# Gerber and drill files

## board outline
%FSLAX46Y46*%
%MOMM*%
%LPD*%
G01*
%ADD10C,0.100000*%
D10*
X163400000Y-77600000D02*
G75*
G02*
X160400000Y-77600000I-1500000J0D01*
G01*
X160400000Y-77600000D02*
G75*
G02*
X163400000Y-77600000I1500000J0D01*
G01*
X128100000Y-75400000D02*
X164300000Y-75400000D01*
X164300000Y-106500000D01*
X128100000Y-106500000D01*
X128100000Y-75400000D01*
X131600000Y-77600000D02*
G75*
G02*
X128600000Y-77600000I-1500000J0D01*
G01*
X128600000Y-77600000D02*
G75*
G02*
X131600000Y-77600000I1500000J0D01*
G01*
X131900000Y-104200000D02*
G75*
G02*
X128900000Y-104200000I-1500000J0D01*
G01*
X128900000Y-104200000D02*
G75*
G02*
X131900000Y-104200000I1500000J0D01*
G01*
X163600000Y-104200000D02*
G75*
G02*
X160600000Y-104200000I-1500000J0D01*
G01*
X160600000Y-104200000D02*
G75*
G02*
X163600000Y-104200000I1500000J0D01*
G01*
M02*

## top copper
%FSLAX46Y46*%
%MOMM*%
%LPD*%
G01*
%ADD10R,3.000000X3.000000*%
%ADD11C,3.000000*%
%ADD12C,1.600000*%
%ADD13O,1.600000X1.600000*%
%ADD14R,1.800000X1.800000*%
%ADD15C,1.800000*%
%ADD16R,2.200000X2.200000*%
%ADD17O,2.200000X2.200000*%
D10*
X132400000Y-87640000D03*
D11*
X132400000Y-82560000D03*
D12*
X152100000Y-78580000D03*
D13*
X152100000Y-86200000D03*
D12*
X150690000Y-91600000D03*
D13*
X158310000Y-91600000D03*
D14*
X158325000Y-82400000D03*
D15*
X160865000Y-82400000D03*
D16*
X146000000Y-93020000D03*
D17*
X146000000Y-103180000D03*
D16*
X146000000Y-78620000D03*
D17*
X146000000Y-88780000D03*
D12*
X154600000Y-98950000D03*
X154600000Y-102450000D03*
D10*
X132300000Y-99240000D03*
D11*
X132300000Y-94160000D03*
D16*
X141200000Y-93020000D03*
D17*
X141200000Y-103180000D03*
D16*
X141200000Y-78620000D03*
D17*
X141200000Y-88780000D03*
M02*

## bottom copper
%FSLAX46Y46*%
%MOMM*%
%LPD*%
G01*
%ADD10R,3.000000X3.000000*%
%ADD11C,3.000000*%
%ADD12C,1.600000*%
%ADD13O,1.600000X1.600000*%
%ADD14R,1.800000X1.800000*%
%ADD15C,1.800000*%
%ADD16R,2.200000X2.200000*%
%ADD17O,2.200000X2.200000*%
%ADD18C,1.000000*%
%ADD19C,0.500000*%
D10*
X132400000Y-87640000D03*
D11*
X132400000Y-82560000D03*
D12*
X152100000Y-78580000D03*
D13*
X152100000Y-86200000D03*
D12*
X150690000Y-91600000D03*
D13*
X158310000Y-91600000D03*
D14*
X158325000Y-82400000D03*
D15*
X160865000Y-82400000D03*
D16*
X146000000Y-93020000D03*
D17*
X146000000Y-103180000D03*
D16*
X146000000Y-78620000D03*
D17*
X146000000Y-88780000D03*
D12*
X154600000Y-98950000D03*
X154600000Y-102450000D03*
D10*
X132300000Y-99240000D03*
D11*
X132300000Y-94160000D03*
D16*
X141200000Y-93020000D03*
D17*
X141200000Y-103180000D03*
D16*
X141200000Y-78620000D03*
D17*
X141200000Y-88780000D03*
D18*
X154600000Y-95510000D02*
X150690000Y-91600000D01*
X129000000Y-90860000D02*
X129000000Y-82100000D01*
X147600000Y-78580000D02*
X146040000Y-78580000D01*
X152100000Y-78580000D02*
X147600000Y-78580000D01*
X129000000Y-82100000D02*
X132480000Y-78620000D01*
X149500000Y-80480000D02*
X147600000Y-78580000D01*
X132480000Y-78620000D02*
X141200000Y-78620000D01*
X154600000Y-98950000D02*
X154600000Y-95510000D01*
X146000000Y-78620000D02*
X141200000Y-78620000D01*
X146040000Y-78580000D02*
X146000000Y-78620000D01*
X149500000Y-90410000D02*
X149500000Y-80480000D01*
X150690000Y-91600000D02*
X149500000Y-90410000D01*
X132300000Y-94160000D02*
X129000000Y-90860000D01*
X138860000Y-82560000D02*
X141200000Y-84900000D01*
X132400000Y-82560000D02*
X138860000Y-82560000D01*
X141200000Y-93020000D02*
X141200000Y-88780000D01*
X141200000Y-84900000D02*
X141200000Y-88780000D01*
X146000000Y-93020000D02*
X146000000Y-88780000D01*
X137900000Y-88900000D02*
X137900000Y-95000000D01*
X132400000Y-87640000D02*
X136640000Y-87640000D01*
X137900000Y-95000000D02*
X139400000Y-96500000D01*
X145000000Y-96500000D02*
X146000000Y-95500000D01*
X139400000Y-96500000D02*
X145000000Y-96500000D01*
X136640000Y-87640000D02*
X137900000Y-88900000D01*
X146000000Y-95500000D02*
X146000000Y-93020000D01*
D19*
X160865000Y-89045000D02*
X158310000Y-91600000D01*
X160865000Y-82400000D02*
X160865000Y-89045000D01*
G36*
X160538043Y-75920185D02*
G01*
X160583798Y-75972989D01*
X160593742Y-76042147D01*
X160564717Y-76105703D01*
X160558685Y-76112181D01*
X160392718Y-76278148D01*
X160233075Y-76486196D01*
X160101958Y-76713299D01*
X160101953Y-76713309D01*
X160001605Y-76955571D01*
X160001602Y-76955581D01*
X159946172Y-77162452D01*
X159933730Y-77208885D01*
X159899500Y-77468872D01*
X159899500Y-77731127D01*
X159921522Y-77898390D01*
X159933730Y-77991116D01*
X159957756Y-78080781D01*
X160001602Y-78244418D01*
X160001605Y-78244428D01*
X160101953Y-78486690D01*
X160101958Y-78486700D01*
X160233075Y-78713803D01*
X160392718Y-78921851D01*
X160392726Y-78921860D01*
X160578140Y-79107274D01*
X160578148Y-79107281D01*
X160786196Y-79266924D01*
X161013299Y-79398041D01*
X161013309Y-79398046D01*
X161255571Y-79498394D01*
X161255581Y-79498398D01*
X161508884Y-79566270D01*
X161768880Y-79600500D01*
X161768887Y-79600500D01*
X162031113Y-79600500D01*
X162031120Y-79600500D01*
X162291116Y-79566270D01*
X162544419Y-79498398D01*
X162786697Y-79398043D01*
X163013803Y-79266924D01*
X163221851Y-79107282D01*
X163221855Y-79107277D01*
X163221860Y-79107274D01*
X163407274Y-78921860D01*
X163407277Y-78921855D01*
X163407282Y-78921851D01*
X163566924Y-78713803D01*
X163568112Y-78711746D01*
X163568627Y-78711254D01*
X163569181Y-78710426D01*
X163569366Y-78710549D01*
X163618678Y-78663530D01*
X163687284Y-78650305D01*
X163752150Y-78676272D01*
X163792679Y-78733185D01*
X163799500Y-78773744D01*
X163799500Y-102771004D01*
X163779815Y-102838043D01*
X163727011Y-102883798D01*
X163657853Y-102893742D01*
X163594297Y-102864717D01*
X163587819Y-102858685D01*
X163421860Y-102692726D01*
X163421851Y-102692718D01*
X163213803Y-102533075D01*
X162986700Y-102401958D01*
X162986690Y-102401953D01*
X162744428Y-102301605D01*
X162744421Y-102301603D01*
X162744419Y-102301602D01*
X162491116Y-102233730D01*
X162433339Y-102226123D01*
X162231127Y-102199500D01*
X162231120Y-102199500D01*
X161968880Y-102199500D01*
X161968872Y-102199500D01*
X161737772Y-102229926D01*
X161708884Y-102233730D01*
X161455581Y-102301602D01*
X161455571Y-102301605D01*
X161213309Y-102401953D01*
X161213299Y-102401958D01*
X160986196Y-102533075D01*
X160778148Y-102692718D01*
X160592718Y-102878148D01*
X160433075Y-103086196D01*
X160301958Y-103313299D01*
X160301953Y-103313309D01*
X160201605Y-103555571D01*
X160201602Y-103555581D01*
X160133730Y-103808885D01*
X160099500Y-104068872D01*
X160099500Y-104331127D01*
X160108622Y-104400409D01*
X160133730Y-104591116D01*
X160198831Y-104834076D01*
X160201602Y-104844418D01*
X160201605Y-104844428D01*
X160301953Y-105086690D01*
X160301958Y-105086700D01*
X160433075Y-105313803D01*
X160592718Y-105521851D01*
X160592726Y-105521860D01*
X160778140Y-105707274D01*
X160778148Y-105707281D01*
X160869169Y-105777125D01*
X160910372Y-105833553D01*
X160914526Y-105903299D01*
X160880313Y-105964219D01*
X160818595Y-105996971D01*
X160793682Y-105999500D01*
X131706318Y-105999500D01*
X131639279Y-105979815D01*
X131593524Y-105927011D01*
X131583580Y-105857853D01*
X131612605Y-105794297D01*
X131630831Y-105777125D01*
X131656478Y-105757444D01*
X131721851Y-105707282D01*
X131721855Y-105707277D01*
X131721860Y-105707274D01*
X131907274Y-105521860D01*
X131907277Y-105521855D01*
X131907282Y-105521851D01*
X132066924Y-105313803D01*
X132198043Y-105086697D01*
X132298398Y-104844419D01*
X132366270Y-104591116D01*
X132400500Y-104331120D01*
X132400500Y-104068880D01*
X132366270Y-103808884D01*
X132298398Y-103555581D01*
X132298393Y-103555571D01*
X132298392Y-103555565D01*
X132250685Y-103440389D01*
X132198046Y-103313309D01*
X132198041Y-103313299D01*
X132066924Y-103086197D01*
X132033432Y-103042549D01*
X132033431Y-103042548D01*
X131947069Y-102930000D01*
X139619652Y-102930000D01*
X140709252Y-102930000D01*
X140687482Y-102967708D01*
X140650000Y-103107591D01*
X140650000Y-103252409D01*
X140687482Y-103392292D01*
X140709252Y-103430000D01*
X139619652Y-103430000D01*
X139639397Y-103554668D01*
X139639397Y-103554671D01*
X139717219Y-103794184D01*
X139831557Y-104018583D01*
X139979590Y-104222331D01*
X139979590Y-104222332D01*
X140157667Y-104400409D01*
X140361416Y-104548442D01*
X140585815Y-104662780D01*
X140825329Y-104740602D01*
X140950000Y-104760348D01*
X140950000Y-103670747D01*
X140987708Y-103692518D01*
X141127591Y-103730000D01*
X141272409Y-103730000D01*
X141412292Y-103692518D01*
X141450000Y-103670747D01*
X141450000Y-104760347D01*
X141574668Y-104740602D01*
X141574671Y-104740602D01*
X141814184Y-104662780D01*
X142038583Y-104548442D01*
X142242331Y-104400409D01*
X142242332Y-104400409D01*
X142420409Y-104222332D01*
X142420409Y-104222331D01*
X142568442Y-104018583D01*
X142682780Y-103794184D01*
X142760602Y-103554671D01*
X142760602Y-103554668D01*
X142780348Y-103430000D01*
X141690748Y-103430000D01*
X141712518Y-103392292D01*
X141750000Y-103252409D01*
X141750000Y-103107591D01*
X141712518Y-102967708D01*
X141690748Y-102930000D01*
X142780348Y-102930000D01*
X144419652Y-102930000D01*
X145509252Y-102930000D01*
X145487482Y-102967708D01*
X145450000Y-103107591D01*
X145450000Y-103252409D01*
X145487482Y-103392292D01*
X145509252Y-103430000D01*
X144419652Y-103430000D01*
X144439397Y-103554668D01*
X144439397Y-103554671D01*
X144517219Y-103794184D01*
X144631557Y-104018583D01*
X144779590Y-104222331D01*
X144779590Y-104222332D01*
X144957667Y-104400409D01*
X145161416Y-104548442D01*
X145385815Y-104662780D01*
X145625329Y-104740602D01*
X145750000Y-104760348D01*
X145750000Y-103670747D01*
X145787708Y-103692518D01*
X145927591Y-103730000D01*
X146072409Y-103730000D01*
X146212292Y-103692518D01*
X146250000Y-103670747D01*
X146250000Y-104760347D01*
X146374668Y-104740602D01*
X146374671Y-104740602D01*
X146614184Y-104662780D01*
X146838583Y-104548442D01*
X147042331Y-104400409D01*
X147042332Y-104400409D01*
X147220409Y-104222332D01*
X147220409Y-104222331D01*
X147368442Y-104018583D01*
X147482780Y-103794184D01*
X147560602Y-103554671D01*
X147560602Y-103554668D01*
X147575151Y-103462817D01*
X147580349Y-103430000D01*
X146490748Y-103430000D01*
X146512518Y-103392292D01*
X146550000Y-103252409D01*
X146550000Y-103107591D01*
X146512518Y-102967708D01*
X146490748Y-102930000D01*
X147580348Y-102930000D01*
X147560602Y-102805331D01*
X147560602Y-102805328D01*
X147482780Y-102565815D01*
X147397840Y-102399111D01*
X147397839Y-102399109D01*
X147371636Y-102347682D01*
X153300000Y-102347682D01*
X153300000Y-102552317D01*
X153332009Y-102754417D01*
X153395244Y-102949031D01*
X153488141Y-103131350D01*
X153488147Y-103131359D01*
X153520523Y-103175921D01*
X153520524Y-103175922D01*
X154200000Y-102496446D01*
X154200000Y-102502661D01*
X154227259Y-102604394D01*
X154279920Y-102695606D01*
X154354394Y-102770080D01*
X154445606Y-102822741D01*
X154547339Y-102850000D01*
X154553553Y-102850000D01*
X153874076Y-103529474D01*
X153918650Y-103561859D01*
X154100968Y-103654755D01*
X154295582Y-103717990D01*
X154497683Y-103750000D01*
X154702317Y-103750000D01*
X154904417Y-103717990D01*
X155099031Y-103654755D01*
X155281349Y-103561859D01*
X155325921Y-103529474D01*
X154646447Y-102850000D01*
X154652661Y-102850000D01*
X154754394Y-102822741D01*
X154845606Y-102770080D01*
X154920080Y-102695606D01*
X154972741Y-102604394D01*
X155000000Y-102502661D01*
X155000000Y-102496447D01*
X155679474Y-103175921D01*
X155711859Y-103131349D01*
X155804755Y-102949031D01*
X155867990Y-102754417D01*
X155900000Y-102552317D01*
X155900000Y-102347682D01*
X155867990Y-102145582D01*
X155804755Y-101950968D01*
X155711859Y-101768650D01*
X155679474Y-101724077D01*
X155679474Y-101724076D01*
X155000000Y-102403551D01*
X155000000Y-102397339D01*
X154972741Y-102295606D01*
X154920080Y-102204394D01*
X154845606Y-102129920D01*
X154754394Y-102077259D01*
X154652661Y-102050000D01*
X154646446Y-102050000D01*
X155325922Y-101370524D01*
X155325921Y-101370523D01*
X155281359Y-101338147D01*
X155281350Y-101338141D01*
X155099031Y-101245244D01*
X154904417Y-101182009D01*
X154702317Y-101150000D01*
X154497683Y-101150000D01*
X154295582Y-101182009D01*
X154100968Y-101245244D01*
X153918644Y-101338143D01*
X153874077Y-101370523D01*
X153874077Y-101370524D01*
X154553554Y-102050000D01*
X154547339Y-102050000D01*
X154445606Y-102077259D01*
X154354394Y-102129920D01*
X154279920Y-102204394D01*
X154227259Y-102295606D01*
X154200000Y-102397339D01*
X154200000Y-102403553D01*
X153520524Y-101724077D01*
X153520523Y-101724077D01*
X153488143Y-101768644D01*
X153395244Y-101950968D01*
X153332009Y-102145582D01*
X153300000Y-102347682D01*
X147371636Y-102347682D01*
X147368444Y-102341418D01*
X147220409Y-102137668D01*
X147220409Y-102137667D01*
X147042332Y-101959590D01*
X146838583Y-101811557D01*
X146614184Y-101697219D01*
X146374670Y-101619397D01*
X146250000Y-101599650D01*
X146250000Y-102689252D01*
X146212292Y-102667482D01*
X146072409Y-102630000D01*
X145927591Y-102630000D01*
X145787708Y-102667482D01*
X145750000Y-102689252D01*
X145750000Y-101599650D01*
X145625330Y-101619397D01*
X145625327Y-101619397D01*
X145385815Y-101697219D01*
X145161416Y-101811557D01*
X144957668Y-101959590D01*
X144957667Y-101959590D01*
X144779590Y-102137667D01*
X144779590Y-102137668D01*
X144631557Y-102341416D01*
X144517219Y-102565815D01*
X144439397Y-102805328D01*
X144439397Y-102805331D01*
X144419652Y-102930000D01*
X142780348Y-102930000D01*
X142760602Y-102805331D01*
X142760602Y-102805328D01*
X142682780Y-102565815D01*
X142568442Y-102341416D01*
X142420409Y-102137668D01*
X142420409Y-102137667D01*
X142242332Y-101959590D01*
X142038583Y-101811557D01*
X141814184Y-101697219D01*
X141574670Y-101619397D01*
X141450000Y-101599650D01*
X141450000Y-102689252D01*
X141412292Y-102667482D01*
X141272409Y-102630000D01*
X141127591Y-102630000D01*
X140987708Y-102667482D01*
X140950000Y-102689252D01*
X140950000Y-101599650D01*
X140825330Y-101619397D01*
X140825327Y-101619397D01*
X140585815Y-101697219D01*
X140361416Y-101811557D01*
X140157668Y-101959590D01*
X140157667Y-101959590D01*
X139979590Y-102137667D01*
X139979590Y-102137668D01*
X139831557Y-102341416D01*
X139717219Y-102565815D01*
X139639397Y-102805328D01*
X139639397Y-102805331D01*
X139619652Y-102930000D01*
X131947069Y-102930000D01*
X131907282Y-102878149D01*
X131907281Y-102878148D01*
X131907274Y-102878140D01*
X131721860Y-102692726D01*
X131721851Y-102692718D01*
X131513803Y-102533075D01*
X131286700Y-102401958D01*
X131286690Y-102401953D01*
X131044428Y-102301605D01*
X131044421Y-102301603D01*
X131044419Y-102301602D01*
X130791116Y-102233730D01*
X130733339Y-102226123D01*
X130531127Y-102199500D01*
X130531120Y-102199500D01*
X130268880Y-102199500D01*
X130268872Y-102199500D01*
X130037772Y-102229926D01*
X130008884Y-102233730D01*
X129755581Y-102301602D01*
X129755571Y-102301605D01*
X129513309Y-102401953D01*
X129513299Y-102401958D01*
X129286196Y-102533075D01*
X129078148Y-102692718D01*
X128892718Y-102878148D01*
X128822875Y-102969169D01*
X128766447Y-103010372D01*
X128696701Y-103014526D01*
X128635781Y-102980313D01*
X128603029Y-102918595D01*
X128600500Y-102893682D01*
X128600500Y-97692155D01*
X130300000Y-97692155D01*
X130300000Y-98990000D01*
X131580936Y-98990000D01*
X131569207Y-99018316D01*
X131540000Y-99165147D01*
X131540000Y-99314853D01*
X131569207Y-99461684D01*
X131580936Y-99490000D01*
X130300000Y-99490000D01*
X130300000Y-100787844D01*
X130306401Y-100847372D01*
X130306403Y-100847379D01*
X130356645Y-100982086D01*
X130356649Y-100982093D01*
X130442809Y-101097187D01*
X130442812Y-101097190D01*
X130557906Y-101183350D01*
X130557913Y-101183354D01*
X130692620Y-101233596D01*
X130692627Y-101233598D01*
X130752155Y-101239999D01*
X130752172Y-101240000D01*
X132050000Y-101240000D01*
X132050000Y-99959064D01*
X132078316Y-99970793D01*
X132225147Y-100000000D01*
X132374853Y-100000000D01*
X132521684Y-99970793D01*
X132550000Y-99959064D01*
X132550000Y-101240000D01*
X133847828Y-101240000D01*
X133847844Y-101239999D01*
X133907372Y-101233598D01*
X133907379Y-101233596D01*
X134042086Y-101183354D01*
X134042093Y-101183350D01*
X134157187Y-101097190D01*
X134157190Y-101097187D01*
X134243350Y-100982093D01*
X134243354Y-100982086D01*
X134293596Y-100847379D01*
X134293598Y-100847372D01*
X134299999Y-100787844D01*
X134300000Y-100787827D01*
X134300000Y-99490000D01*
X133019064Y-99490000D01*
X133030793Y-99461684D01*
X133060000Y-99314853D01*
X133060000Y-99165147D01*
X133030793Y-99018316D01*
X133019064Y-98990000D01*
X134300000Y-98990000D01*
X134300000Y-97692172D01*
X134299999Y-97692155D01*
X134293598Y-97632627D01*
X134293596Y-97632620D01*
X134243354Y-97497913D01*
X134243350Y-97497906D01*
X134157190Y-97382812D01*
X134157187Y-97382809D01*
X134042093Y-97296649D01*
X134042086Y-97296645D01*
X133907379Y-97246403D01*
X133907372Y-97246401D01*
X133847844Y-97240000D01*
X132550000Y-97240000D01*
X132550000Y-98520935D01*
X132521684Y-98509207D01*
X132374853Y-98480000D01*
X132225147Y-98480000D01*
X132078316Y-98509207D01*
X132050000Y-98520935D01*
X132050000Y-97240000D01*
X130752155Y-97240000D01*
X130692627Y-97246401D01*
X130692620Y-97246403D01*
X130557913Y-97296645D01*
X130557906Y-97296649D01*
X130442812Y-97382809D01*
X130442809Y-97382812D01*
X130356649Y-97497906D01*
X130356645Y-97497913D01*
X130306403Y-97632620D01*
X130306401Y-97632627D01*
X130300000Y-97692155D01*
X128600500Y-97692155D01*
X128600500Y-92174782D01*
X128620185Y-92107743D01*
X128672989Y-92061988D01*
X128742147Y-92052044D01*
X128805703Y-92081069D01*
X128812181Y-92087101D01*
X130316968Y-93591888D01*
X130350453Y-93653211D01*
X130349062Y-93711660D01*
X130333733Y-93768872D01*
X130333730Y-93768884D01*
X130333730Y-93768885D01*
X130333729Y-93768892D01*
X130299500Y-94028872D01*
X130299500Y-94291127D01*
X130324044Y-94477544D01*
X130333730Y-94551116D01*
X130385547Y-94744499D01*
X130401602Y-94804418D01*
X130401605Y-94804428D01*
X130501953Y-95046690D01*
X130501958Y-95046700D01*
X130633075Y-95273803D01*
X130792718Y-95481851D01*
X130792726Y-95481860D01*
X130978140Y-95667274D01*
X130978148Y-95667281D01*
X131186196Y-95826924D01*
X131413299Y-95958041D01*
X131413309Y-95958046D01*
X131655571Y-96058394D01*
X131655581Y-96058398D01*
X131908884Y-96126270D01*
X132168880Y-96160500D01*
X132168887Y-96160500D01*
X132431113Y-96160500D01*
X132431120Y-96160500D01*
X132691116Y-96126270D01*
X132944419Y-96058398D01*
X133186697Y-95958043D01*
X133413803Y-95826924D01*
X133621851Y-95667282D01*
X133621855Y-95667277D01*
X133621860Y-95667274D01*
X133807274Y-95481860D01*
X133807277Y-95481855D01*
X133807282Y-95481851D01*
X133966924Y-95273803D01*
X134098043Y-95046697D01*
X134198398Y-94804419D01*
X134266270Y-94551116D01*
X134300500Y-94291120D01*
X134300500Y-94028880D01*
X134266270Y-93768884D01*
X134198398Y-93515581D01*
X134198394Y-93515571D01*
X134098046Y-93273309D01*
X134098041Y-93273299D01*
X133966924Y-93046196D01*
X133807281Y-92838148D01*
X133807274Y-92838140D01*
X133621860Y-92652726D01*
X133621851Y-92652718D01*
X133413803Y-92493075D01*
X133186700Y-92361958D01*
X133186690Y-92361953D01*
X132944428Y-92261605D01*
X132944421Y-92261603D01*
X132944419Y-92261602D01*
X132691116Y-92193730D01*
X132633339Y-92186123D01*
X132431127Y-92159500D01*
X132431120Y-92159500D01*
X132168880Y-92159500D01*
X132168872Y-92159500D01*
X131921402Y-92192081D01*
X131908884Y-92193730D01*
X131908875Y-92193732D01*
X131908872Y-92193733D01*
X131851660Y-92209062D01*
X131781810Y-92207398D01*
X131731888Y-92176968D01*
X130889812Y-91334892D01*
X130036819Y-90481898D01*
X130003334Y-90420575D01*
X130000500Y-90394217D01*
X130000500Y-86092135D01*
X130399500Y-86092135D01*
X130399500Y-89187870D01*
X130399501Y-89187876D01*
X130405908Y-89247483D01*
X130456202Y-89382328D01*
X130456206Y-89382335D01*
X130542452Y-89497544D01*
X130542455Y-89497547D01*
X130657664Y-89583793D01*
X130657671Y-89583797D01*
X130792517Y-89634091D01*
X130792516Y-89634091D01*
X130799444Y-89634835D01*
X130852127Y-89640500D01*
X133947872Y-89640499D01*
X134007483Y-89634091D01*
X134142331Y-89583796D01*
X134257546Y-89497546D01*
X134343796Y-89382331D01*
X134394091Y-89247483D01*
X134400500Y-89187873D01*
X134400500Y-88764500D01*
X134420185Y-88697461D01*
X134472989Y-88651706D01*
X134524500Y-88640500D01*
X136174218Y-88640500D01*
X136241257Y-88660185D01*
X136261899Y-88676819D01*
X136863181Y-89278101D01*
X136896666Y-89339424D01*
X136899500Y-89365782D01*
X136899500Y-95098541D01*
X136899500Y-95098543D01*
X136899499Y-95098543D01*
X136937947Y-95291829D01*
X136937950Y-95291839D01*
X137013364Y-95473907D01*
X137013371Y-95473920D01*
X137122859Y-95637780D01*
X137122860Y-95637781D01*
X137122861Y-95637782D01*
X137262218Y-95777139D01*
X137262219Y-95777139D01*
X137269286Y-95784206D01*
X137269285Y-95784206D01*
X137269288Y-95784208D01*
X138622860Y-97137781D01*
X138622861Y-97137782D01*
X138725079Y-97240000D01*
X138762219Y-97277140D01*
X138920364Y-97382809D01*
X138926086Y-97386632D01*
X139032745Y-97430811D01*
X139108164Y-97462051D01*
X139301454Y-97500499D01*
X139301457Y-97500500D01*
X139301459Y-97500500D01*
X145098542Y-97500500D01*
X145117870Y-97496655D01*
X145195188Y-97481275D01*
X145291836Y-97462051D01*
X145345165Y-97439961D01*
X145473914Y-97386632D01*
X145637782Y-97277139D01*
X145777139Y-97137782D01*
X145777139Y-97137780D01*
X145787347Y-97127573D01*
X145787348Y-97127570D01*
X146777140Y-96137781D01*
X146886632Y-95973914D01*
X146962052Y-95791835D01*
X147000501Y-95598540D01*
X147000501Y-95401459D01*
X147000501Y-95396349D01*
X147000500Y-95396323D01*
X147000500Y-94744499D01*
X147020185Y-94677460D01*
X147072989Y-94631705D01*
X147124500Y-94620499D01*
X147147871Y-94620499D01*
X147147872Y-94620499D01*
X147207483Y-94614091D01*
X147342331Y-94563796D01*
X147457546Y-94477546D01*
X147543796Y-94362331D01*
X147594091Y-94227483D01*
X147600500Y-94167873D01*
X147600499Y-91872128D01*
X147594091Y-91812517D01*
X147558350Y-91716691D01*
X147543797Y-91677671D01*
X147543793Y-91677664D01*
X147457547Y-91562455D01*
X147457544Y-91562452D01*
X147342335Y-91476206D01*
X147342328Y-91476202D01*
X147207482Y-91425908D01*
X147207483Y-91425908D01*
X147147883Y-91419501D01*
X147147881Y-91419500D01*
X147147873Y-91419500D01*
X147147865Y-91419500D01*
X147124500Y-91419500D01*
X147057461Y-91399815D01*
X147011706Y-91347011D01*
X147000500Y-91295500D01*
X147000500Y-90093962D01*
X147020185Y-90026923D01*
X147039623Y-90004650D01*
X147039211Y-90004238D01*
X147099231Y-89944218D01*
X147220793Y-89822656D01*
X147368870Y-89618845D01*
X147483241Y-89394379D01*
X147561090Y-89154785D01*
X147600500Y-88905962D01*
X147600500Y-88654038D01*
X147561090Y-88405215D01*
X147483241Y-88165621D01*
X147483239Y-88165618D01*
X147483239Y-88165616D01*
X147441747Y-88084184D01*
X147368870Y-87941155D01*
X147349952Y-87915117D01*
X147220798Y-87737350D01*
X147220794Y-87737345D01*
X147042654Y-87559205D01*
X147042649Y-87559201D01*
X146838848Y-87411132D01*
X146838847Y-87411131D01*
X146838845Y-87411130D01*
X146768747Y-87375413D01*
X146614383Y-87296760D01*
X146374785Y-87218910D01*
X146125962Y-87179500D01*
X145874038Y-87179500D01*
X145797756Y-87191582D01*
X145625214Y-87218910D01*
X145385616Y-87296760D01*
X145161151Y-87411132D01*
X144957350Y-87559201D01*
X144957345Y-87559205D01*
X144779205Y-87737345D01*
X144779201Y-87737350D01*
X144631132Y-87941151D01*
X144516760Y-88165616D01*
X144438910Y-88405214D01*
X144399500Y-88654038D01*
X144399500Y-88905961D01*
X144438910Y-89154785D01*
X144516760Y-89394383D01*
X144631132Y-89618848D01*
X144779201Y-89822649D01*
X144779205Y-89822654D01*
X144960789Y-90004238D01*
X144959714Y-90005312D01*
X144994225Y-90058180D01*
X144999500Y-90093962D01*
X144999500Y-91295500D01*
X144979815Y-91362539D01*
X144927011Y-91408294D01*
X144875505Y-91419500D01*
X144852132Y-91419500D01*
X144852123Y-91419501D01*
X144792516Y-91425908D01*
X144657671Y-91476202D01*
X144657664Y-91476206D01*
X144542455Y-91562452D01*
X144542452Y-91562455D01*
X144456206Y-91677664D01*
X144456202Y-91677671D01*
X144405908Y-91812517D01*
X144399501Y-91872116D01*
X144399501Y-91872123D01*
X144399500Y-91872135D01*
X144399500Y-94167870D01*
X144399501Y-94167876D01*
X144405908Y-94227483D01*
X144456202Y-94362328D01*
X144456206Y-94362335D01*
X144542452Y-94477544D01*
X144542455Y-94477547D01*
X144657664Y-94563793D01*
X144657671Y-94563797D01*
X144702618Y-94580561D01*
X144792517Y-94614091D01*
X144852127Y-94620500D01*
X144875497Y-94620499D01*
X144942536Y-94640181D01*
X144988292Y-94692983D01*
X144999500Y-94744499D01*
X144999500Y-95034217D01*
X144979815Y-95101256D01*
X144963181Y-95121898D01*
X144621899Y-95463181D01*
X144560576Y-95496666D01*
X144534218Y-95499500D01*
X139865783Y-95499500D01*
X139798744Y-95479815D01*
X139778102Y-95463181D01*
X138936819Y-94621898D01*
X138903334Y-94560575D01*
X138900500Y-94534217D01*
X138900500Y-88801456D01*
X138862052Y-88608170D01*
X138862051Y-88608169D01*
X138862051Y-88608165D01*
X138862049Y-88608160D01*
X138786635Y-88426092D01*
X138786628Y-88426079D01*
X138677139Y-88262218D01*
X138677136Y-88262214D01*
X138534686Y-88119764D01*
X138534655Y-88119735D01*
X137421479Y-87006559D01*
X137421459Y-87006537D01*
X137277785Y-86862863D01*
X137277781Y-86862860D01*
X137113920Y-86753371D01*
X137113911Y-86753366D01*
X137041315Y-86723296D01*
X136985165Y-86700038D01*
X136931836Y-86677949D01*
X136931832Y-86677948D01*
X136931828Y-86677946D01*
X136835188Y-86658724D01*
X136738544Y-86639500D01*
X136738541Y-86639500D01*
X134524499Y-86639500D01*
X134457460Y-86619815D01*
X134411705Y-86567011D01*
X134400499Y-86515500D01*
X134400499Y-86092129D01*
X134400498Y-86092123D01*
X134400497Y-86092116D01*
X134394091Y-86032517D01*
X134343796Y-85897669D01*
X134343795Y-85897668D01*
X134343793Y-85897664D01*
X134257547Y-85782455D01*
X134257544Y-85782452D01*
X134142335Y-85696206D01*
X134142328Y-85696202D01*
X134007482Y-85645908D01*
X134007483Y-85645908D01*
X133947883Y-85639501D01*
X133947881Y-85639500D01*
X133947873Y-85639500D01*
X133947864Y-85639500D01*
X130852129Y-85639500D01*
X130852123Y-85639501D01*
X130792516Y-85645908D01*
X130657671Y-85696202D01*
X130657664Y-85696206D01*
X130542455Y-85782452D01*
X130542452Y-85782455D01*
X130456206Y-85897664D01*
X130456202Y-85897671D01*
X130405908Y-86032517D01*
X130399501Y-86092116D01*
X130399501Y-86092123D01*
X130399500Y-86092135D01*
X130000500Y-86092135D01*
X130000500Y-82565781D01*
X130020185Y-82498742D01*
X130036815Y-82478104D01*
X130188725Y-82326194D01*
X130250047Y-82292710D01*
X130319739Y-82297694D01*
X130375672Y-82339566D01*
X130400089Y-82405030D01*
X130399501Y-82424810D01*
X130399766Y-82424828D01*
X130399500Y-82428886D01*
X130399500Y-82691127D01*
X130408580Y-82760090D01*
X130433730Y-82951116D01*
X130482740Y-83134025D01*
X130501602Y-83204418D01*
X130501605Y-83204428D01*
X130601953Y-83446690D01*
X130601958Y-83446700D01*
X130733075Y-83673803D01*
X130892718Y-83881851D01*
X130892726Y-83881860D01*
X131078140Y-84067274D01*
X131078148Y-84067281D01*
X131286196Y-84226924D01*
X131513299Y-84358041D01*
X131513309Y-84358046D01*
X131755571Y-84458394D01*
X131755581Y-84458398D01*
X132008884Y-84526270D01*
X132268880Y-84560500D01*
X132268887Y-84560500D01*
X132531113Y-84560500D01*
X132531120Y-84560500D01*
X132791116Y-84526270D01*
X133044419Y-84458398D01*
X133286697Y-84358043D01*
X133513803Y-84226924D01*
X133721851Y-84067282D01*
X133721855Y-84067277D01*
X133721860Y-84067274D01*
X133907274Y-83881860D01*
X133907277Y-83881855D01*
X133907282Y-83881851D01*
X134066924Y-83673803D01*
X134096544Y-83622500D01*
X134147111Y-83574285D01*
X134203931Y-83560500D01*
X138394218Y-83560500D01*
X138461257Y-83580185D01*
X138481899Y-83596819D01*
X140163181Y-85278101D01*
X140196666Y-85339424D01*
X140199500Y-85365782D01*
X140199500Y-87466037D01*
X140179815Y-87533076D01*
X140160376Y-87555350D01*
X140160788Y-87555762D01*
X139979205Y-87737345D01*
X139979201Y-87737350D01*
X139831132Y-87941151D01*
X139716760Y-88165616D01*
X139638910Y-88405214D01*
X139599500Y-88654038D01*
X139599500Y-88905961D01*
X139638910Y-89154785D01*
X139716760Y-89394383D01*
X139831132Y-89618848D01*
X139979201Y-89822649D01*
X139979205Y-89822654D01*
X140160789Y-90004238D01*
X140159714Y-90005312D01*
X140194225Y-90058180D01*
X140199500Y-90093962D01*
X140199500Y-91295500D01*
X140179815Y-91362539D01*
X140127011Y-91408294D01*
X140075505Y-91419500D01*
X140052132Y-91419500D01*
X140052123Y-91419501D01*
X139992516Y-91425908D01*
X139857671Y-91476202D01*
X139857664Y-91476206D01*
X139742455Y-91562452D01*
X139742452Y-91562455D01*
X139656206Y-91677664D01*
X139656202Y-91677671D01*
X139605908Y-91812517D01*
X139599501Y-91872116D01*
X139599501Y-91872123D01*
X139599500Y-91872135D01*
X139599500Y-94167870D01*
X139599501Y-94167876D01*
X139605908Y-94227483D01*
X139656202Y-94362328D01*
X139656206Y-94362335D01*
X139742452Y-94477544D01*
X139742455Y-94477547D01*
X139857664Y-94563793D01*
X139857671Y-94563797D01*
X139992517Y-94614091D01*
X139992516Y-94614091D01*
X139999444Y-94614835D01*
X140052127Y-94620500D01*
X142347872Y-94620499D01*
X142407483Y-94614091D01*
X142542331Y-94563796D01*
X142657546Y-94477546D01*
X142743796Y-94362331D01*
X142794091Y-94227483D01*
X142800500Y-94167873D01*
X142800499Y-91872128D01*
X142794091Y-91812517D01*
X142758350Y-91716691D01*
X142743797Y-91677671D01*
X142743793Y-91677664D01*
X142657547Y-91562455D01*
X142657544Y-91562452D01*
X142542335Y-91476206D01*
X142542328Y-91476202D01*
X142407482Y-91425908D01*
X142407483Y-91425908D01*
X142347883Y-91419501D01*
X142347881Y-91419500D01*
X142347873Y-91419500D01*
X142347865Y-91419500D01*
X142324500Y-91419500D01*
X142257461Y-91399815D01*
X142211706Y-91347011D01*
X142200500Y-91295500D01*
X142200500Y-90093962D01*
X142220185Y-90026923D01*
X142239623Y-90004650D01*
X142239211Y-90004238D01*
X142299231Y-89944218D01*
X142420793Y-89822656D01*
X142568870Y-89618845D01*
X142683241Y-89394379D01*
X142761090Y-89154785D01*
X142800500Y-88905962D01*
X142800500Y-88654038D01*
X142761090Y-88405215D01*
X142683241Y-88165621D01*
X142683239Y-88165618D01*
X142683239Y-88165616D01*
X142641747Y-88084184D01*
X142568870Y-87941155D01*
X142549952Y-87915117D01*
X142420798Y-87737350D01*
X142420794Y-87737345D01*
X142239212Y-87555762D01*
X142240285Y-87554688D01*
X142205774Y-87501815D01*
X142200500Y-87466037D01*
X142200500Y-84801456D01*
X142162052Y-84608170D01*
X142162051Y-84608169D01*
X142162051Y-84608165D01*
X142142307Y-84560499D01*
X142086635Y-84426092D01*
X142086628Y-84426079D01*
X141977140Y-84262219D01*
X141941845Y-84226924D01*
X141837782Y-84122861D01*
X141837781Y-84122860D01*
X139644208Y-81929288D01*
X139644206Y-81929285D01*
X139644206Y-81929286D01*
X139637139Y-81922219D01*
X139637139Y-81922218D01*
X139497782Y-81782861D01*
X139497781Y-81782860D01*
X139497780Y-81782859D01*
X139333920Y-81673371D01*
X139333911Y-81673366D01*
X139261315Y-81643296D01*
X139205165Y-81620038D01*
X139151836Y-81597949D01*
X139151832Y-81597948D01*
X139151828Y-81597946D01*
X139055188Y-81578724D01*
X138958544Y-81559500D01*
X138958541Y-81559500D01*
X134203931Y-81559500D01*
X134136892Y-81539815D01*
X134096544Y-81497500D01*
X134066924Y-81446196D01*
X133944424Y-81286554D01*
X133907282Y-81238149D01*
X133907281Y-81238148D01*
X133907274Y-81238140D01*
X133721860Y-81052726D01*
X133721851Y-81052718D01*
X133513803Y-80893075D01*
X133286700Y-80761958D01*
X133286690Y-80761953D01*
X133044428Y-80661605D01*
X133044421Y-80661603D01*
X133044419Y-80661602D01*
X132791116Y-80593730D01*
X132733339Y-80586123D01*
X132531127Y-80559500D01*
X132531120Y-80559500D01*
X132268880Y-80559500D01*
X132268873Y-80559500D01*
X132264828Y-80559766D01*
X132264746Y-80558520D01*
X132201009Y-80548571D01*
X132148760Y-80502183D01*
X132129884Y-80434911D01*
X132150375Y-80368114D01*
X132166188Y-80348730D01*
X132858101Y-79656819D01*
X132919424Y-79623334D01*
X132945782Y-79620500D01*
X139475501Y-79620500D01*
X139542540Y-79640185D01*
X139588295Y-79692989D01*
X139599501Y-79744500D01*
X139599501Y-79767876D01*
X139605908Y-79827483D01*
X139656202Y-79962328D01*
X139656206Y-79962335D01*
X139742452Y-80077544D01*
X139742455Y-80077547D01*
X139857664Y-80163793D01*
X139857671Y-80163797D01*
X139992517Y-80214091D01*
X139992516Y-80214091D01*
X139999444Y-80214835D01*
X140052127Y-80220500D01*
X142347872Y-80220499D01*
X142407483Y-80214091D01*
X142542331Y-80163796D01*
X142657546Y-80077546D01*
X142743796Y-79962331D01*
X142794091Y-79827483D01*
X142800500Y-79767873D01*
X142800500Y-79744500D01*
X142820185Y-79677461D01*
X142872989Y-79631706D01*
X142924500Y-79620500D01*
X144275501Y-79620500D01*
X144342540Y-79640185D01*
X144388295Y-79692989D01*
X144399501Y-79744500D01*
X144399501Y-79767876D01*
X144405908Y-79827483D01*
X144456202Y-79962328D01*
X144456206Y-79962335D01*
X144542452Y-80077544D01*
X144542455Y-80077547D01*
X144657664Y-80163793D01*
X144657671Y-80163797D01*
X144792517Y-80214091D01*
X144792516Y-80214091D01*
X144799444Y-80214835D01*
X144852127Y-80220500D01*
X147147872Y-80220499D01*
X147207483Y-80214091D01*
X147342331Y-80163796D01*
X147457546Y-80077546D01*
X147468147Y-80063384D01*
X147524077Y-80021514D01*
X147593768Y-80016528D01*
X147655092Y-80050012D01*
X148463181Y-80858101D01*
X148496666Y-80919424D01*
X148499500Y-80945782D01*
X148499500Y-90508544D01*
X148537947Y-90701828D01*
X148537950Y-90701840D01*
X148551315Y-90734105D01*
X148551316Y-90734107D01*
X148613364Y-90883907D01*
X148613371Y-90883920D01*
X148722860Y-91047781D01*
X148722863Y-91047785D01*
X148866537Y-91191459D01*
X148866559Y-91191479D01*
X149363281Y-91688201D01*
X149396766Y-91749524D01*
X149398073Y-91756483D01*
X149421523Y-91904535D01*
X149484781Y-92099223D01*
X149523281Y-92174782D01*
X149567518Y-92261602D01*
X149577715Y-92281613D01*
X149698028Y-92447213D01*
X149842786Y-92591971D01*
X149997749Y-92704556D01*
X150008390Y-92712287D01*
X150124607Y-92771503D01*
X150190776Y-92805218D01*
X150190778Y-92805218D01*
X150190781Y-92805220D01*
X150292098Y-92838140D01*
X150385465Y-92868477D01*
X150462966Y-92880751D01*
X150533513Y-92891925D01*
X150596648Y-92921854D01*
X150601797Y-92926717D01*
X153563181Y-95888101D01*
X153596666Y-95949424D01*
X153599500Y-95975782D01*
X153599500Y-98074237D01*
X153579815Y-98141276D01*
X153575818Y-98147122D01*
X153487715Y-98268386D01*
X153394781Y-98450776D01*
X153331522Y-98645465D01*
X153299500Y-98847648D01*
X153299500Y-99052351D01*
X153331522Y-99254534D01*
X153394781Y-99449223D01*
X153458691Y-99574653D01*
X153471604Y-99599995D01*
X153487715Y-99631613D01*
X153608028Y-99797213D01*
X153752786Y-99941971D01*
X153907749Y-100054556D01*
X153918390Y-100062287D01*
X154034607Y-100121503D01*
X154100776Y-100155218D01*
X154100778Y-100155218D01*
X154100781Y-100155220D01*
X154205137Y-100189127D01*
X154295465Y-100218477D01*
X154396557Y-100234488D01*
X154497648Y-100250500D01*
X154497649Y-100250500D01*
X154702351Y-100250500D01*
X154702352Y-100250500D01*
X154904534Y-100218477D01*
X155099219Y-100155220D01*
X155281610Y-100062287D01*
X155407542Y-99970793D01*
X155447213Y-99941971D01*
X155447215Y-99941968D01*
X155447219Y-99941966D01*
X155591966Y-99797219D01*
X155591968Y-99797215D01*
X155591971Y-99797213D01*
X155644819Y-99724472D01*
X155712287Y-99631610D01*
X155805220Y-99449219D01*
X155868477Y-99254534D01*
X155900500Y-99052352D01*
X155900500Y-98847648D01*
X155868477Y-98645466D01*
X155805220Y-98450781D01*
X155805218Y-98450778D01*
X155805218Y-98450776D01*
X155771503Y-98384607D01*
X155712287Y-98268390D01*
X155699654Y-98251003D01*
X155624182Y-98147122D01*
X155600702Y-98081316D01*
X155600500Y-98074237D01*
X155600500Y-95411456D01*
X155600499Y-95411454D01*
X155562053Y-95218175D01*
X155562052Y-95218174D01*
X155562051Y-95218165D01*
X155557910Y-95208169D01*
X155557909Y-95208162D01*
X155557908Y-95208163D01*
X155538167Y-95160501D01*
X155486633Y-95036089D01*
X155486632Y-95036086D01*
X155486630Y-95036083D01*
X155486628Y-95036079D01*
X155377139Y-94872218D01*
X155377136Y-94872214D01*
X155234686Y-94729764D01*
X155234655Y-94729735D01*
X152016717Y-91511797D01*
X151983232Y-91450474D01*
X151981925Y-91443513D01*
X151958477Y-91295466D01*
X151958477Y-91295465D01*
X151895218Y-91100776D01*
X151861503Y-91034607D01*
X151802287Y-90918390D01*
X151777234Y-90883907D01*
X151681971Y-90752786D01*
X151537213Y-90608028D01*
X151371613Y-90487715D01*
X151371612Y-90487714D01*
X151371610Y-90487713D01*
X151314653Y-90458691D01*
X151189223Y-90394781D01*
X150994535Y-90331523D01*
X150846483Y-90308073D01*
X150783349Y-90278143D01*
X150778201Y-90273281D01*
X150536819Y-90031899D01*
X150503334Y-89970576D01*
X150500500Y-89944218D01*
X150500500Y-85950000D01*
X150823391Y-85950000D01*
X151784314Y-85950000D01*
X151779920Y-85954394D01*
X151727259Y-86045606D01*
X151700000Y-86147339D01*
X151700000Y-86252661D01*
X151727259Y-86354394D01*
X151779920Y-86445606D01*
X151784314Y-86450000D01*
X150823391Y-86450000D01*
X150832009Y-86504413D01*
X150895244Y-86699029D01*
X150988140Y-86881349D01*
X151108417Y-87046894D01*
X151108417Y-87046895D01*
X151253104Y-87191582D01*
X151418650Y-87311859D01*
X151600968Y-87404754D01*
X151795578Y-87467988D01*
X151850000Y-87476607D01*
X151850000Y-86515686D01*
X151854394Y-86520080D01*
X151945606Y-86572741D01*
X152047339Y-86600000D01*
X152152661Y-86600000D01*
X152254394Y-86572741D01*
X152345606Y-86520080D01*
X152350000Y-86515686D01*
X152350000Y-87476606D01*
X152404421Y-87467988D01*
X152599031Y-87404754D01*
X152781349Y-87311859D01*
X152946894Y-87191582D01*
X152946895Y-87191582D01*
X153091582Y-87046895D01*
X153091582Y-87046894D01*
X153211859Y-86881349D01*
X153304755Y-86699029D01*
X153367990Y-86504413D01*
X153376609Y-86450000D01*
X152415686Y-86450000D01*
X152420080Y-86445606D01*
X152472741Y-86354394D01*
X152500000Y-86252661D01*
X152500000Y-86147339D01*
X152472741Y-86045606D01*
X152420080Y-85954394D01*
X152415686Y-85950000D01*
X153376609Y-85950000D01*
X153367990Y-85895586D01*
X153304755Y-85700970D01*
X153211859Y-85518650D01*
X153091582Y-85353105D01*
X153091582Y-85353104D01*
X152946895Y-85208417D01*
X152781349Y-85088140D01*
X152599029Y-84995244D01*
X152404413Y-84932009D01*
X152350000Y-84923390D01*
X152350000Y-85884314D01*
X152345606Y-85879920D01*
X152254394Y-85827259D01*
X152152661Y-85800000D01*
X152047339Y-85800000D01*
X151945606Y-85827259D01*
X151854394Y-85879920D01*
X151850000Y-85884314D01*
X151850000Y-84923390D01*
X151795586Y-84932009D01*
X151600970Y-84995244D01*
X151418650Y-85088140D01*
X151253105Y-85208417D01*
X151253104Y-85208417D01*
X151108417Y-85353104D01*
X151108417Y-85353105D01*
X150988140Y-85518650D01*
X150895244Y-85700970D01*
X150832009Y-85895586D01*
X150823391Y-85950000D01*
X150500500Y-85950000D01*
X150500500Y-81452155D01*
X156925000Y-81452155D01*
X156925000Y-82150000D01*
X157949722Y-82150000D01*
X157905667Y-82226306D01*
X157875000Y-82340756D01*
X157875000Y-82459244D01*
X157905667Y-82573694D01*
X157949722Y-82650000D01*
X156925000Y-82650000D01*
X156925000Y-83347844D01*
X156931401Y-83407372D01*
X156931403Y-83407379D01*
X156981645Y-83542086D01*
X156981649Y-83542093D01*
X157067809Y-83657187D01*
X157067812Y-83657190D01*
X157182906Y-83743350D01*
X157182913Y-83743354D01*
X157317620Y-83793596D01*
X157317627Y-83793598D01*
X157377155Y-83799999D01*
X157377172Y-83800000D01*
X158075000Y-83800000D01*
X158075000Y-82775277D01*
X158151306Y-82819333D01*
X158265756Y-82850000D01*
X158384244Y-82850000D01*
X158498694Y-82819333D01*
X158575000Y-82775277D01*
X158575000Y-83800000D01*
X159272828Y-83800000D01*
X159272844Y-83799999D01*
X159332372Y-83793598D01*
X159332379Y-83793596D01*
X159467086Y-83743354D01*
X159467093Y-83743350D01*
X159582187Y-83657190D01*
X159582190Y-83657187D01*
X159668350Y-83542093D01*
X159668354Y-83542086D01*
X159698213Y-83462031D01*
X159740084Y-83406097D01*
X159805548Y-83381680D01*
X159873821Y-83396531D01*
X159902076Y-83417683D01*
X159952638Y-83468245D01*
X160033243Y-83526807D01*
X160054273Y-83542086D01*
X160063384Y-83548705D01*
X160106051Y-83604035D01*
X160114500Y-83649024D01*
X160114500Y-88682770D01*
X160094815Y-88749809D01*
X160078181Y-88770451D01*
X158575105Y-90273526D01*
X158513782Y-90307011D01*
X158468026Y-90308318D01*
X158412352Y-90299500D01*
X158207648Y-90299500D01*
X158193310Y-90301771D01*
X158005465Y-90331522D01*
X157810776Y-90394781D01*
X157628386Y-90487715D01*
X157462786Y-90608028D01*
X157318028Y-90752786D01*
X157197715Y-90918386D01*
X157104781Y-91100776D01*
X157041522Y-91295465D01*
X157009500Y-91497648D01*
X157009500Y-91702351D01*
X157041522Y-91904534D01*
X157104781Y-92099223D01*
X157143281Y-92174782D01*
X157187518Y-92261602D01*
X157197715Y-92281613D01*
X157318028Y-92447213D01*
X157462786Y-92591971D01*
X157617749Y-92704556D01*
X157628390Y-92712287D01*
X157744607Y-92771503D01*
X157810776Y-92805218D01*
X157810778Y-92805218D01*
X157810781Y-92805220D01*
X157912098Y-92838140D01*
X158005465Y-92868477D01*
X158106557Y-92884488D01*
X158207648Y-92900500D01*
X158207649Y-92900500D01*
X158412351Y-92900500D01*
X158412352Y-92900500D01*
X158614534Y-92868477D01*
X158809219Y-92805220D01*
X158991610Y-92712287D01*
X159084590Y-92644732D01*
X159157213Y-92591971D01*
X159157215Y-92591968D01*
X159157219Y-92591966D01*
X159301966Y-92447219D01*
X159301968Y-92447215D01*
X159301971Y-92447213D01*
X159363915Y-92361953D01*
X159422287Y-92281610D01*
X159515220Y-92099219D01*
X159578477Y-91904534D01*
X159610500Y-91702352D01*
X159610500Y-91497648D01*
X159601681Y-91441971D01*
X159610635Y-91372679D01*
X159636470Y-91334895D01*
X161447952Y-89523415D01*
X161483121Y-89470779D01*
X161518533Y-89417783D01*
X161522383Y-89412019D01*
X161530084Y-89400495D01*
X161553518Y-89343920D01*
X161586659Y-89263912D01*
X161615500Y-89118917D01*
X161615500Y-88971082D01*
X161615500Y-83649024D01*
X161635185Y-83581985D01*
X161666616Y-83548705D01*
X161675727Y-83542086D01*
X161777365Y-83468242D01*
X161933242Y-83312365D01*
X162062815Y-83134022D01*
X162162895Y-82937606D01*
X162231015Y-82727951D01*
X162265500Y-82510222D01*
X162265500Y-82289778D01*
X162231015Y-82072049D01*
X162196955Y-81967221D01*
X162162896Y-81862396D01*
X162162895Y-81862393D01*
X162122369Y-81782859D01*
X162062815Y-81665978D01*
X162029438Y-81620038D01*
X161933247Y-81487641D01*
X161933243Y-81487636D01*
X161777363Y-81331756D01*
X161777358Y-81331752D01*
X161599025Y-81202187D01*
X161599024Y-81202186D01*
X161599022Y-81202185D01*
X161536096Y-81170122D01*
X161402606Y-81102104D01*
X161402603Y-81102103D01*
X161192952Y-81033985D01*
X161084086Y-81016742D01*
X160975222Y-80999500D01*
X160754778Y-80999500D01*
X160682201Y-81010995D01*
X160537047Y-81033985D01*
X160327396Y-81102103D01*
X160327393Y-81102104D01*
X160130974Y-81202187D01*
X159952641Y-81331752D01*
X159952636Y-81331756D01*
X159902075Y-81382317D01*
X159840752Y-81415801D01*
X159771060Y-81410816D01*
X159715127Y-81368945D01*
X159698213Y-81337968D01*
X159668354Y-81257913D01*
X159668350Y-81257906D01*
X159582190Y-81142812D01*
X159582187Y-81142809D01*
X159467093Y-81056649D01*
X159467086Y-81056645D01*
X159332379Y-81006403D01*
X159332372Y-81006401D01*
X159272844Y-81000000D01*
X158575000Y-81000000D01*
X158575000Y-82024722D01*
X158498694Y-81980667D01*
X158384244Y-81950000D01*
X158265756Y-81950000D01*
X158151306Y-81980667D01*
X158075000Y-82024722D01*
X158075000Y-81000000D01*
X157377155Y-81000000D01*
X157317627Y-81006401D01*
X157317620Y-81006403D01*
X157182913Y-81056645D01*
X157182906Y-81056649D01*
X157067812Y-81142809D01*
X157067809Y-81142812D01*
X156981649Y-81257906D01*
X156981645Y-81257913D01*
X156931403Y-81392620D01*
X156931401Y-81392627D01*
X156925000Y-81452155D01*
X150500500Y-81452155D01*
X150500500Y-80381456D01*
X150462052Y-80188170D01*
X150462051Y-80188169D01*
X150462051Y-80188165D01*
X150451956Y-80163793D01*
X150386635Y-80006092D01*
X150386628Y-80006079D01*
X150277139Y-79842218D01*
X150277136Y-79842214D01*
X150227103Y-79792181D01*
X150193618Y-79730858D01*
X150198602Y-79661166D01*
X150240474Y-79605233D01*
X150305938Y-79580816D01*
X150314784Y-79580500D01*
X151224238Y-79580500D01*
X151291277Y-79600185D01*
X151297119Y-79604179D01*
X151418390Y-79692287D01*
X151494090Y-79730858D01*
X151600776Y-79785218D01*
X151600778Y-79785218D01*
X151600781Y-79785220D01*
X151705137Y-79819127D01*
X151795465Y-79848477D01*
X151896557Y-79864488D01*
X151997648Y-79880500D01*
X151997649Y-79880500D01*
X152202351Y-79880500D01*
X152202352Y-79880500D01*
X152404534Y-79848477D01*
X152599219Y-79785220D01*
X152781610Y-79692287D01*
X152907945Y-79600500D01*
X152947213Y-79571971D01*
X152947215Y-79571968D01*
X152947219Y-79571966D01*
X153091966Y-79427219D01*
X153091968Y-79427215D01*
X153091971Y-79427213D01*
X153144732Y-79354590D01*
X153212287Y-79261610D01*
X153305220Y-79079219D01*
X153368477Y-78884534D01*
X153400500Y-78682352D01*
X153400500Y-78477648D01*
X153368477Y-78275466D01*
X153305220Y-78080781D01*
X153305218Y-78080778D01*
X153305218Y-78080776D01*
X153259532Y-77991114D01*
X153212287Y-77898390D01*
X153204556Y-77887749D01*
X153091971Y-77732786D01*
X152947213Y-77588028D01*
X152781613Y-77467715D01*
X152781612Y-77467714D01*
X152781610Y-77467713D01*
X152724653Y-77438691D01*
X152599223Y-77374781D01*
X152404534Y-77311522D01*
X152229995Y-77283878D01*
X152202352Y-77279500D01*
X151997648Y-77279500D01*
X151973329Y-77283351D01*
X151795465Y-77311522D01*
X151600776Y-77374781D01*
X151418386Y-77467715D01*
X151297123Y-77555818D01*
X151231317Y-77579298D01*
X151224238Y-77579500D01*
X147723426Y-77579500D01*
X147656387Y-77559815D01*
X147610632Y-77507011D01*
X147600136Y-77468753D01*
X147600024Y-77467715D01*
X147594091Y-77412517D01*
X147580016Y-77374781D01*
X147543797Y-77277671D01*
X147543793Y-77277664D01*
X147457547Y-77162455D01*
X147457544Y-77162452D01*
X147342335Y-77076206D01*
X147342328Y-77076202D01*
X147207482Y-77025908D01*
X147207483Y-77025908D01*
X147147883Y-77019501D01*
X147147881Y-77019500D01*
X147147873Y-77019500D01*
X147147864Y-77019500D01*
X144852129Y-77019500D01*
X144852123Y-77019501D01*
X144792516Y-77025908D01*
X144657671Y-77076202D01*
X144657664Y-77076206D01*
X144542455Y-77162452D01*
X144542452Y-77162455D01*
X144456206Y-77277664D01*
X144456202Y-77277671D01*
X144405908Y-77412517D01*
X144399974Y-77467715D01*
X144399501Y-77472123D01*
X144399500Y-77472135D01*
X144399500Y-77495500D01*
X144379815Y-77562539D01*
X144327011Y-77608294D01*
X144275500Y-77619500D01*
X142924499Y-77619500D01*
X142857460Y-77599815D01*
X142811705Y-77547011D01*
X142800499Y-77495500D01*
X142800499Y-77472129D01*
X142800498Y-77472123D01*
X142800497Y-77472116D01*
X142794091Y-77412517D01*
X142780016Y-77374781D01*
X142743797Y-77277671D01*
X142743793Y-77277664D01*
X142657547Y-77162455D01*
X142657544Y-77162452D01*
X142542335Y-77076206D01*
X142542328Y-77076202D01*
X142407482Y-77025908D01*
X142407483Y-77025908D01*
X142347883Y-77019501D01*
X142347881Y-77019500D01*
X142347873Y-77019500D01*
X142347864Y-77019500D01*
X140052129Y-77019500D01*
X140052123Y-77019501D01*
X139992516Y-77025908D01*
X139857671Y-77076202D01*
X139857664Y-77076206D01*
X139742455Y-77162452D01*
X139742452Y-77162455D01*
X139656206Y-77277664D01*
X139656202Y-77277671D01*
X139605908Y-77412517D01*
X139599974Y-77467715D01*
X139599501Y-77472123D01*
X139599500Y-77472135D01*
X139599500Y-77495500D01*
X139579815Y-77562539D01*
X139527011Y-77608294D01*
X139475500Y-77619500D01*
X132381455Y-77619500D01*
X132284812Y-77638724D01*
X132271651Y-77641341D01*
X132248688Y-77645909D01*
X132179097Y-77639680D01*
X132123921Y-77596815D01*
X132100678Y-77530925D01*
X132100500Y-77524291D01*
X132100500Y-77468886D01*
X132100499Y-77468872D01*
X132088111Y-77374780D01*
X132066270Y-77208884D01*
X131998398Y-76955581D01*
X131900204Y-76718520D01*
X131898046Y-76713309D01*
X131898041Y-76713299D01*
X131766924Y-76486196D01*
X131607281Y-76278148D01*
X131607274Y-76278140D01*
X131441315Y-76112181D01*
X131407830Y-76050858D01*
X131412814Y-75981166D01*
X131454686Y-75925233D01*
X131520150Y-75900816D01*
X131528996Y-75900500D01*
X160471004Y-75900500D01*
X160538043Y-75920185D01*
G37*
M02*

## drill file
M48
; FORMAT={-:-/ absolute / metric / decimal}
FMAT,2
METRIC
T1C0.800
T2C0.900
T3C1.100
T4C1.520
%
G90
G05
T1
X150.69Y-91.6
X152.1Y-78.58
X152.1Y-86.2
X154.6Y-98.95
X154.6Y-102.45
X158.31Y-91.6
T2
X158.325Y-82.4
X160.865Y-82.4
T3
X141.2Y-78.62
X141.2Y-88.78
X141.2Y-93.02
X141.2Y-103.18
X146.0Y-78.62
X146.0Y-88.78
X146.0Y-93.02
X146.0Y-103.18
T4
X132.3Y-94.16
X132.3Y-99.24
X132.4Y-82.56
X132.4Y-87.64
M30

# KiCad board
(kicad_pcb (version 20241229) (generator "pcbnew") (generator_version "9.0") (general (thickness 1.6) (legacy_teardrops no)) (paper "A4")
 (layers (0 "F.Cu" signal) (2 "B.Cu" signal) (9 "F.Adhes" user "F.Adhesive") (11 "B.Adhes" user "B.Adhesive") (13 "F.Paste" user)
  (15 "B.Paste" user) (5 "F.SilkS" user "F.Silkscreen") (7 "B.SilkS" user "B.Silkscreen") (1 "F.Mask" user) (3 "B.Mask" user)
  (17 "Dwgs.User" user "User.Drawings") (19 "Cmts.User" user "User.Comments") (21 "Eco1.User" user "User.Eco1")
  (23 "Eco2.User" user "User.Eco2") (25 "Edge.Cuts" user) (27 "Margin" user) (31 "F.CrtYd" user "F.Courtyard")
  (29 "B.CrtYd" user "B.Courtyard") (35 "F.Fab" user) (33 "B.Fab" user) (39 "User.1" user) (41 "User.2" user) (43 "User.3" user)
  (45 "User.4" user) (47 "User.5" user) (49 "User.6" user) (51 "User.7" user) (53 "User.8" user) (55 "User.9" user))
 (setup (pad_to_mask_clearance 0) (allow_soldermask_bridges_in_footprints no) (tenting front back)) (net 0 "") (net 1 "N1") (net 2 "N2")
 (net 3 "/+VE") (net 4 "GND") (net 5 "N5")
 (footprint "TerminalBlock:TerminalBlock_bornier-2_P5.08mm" (layer "F.Cu") (at 132.4 87.64 90)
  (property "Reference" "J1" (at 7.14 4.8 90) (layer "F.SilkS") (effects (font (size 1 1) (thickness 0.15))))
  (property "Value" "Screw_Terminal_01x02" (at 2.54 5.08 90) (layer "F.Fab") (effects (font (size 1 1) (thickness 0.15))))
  (pad "1" thru_hole rect (at 0 0 90) (size 3 3) (drill 1.52) (layers "*.Cu" "*.Mask") (remove_unused_layers no) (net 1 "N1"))
  (pad "2" thru_hole circle (at 5.08 0 90) (size 3 3) (drill 1.52) (layers "*.Cu" "*.Mask") (remove_unused_layers no) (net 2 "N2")))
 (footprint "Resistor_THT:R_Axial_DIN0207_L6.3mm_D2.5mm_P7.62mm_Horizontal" (layer "F.Cu") (at 152.1 78.58 -90)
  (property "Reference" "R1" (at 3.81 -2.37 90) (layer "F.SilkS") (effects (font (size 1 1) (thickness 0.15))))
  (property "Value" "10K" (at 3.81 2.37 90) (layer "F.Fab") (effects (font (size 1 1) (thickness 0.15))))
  (pad "1" thru_hole circle (at 0 0 270) (size 1.6 1.6) (drill 0.8) (layers "*.Cu" "*.Mask") (remove_unused_layers no) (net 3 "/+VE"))
  (pad "2" thru_hole oval (at 7.62 0 270) (size 1.6 1.6) (drill 0.8) (layers "*.Cu" "*.Mask") (remove_unused_layers no) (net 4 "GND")))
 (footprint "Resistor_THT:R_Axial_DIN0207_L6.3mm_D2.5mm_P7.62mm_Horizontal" (layer "F.Cu") (at 150.69 91.6)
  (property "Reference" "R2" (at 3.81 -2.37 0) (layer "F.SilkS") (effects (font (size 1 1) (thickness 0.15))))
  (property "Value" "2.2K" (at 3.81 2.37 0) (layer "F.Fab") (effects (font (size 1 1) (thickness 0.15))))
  (pad "1" thru_hole circle (at 0 0) (size 1.6 1.6) (drill 0.8) (layers "*.Cu" "*.Mask") (remove_unused_layers no) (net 3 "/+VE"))
  (pad "2" thru_hole oval (at 7.62 0) (size 1.6 1.6) (drill 0.8) (layers "*.Cu" "*.Mask") (remove_unused_layers no) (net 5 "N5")))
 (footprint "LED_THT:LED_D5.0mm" (layer "F.Cu") (at 158.325 82.4)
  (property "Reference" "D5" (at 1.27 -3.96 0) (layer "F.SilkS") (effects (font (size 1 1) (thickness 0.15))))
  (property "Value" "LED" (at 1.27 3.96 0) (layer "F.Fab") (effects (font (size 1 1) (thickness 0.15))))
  (pad "1" thru_hole rect (at 0 0) (size 1.8 1.8) (drill 0.9) (layers "*.Cu" "*.Mask") (remove_unused_layers no) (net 4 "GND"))
  (pad "2" thru_hole circle (at 2.54 0) (size 1.8 1.8) (drill 0.9) (layers "*.Cu" "*.Mask") (remove_unused_layers no) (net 5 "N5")))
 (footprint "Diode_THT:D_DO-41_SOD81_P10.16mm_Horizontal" (layer "F.Cu") (at 146 93.02 -90)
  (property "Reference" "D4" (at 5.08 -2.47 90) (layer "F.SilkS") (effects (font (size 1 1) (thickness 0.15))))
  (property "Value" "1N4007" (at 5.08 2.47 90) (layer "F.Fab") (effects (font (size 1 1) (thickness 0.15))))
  (pad "1" thru_hole rect (at 0 0 270) (size 2.2 2.2) (drill 1.1) (layers "*.Cu" "*.Mask") (remove_unused_layers no) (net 1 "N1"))
  (pad "2" thru_hole oval (at 10.16 0 270) (size 2.2 2.2) (drill 1.1) (layers "*.Cu" "*.Mask") (remove_unused_layers no) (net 4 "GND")))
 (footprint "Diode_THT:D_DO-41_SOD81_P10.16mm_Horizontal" (layer "F.Cu") (at 146 78.62 -90)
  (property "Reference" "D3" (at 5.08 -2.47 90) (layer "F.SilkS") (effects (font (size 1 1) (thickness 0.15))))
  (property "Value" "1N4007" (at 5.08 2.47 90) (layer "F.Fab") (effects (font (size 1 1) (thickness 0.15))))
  (pad "1" thru_hole rect (at 0 0 270) (size 2.2 2.2) (drill 1.1) (layers "*.Cu" "*.Mask") (remove_unused_layers no) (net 3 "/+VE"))
  (pad "2" thru_hole oval (at 10.16 0 270) (size 2.2 2.2) (drill 1.1) (layers "*.Cu" "*.Mask") (remove_unused_layers no) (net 1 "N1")))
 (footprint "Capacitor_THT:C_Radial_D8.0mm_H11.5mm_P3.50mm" (layer "F.Cu") (at 154.6 98.95 -90)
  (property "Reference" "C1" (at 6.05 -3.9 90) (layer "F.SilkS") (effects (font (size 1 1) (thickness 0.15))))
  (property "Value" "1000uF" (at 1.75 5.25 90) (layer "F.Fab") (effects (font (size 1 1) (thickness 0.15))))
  (pad "1" thru_hole circle (at 0 0 270) (size 1.6 1.6) (drill 0.8) (layers "*.Cu" "*.Mask") (remove_unused_layers no) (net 3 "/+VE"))
  (pad "2" thru_hole circle (at 3.5 0 270) (size 1.6 1.6) (drill 0.8) (layers "*.Cu" "*.Mask") (remove_unused_layers no) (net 4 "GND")))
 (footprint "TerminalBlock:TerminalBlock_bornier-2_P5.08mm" (layer "F.Cu") (at 132.3 99.24 90)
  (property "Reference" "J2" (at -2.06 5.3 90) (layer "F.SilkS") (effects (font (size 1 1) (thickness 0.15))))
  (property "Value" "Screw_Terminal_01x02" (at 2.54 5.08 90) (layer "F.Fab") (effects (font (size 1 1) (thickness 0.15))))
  (pad "1" thru_hole rect (at 0 0 90) (size 3 3) (drill 1.52) (layers "*.Cu" "*.Mask") (remove_unused_layers no) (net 4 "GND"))
  (pad "2" thru_hole circle (at 5.08 0 90) (size 3 3) (drill 1.52) (layers "*.Cu" "*.Mask") (remove_unused_layers no) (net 3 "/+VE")))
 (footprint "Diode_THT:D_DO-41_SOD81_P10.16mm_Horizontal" (layer "F.Cu") (at 141.2 93.02 -90)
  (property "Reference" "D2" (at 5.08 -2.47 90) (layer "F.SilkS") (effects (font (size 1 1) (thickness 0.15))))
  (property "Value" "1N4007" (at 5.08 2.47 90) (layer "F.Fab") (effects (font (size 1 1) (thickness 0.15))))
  (pad "1" thru_hole rect (at 0 0 270) (size 2.2 2.2) (drill 1.1) (layers "*.Cu" "*.Mask") (remove_unused_layers no) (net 2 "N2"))
  (pad "2" thru_hole oval (at 10.16 0 270) (size 2.2 2.2) (drill 1.1) (layers "*.Cu" "*.Mask") (remove_unused_layers no) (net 4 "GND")))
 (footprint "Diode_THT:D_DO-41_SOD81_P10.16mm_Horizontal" (layer "F.Cu") (at 141.2 78.62 -90)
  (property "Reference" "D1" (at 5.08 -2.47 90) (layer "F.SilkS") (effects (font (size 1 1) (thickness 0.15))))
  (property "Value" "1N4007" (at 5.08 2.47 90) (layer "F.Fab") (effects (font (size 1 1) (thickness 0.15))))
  (pad "1" thru_hole rect (at 0 0 270) (size 2.2 2.2) (drill 1.1) (layers "*.Cu" "*.Mask") (remove_unused_layers no) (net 3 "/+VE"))
  (pad "2" thru_hole oval (at 10.16 0 270) (size 2.2 2.2) (drill 1.1) (layers "*.Cu" "*.Mask") (remove_unused_layers no) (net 2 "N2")))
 (gr_circle (center 161.9 77.6) (end 163.4 77.6) (stroke (width 0.1) (type default)) (fill no) (layer "Edge.Cuts"))
 (gr_rect (start 128.1 75.4) (end 164.3 106.5) (stroke (width 0.1) (type default)) (fill no) (layer "Edge.Cuts"))
 (gr_circle (center 130.1 77.6) (end 131.6 77.6) (stroke (width 0.1) (type default)) (fill no) (layer "Edge.Cuts"))
 (gr_circle (center 130.4 104.2) (end 131.9 104.2) (stroke (width 0.1) (type default)) (fill no) (layer "Edge.Cuts"))
 (gr_circle (center 162.1 104.2) (end 163.6 104.2) (stroke (width 0.1) (type default)) (fill no) (layer "Edge.Cuts"))
 (segment (start 154.6 95.51) (end 150.69 91.6) (width 1) (layer "B.Cu") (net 3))
 (segment (start 129 90.86) (end 129 82.1) (width 1) (layer "B.Cu") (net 3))
 (segment (start 147.6 78.58) (end 146.04 78.58) (width 1) (layer "B.Cu") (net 3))
 (segment (start 152.1 78.58) (end 147.6 78.58) (width 1) (layer "B.Cu") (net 3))
 (segment (start 129 82.1) (end 132.48 78.62) (width 1) (layer "B.Cu") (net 3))
 (segment (start 149.5 80.48) (end 147.6 78.58) (width 1) (layer "B.Cu") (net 3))
 (segment (start 132.48 78.62) (end 141.2 78.62) (width 1) (layer "B.Cu") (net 3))
 (segment (start 154.6 98.95) (end 154.6 95.51) (width 1) (layer "B.Cu") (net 3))
 (segment (start 146 78.62) (end 141.2 78.62) (width 1) (layer "B.Cu") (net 3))
 (segment (start 146.04 78.58) (end 146 78.62) (width 1) (layer "B.Cu") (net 3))
 (segment (start 149.5 90.41) (end 149.5 80.48) (width 1) (layer "B.Cu") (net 3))
 (segment (start 150.69 91.6) (end 149.5 90.41) (width 1) (layer "B.Cu") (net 3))
 (segment (start 132.3 94.16) (end 129 90.86) (width 1) (layer "B.Cu") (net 3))
 (segment (start 138.86 82.56) (end 141.2 84.9) (width 1) (layer "B.Cu") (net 2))
 (segment (start 132.4 82.56) (end 138.86 82.56) (width 1) (layer "B.Cu") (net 2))
 (segment (start 141.2 93.02) (end 141.2 88.78) (width 1) (layer "B.Cu") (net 2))
 (segment (start 141.2 84.9) (end 141.2 88.78) (width 1) (layer "B.Cu") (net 2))
 (segment (start 146 93.02) (end 146 88.78) (width 1) (layer "B.Cu") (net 1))
 (segment (start 137.9 88.9) (end 137.9 95) (width 1) (layer "B.Cu") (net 1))
 (segment (start 132.4 87.64) (end 136.64 87.64) (width 1) (layer "B.Cu") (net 1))
 (segment (start 137.9 95) (end 139.4 96.5) (width 1) (layer "B.Cu") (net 1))
 (segment (start 145 96.5) (end 146 95.5) (width 1) (layer "B.Cu") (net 1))
 (segment (start 139.4 96.5) (end 145 96.5) (width 1) (layer "B.Cu") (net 1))
 (segment (start 136.64 87.64) (end 137.9 88.9) (width 1) (layer "B.Cu") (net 1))
 (segment (start 146 95.5) (end 146 93.02) (width 1) (layer "B.Cu") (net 1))
 (segment (start 160.865 89.045) (end 158.31 91.6) (width 0.5) (layer "B.Cu") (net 5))
 (segment (start 160.865 82.4) (end 160.865 89.045) (width 0.5) (layer "B.Cu") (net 5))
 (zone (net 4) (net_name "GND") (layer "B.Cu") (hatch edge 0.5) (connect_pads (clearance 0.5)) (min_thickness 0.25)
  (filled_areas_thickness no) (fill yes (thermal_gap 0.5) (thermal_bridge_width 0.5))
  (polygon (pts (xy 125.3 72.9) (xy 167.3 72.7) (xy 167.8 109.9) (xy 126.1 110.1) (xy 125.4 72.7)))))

